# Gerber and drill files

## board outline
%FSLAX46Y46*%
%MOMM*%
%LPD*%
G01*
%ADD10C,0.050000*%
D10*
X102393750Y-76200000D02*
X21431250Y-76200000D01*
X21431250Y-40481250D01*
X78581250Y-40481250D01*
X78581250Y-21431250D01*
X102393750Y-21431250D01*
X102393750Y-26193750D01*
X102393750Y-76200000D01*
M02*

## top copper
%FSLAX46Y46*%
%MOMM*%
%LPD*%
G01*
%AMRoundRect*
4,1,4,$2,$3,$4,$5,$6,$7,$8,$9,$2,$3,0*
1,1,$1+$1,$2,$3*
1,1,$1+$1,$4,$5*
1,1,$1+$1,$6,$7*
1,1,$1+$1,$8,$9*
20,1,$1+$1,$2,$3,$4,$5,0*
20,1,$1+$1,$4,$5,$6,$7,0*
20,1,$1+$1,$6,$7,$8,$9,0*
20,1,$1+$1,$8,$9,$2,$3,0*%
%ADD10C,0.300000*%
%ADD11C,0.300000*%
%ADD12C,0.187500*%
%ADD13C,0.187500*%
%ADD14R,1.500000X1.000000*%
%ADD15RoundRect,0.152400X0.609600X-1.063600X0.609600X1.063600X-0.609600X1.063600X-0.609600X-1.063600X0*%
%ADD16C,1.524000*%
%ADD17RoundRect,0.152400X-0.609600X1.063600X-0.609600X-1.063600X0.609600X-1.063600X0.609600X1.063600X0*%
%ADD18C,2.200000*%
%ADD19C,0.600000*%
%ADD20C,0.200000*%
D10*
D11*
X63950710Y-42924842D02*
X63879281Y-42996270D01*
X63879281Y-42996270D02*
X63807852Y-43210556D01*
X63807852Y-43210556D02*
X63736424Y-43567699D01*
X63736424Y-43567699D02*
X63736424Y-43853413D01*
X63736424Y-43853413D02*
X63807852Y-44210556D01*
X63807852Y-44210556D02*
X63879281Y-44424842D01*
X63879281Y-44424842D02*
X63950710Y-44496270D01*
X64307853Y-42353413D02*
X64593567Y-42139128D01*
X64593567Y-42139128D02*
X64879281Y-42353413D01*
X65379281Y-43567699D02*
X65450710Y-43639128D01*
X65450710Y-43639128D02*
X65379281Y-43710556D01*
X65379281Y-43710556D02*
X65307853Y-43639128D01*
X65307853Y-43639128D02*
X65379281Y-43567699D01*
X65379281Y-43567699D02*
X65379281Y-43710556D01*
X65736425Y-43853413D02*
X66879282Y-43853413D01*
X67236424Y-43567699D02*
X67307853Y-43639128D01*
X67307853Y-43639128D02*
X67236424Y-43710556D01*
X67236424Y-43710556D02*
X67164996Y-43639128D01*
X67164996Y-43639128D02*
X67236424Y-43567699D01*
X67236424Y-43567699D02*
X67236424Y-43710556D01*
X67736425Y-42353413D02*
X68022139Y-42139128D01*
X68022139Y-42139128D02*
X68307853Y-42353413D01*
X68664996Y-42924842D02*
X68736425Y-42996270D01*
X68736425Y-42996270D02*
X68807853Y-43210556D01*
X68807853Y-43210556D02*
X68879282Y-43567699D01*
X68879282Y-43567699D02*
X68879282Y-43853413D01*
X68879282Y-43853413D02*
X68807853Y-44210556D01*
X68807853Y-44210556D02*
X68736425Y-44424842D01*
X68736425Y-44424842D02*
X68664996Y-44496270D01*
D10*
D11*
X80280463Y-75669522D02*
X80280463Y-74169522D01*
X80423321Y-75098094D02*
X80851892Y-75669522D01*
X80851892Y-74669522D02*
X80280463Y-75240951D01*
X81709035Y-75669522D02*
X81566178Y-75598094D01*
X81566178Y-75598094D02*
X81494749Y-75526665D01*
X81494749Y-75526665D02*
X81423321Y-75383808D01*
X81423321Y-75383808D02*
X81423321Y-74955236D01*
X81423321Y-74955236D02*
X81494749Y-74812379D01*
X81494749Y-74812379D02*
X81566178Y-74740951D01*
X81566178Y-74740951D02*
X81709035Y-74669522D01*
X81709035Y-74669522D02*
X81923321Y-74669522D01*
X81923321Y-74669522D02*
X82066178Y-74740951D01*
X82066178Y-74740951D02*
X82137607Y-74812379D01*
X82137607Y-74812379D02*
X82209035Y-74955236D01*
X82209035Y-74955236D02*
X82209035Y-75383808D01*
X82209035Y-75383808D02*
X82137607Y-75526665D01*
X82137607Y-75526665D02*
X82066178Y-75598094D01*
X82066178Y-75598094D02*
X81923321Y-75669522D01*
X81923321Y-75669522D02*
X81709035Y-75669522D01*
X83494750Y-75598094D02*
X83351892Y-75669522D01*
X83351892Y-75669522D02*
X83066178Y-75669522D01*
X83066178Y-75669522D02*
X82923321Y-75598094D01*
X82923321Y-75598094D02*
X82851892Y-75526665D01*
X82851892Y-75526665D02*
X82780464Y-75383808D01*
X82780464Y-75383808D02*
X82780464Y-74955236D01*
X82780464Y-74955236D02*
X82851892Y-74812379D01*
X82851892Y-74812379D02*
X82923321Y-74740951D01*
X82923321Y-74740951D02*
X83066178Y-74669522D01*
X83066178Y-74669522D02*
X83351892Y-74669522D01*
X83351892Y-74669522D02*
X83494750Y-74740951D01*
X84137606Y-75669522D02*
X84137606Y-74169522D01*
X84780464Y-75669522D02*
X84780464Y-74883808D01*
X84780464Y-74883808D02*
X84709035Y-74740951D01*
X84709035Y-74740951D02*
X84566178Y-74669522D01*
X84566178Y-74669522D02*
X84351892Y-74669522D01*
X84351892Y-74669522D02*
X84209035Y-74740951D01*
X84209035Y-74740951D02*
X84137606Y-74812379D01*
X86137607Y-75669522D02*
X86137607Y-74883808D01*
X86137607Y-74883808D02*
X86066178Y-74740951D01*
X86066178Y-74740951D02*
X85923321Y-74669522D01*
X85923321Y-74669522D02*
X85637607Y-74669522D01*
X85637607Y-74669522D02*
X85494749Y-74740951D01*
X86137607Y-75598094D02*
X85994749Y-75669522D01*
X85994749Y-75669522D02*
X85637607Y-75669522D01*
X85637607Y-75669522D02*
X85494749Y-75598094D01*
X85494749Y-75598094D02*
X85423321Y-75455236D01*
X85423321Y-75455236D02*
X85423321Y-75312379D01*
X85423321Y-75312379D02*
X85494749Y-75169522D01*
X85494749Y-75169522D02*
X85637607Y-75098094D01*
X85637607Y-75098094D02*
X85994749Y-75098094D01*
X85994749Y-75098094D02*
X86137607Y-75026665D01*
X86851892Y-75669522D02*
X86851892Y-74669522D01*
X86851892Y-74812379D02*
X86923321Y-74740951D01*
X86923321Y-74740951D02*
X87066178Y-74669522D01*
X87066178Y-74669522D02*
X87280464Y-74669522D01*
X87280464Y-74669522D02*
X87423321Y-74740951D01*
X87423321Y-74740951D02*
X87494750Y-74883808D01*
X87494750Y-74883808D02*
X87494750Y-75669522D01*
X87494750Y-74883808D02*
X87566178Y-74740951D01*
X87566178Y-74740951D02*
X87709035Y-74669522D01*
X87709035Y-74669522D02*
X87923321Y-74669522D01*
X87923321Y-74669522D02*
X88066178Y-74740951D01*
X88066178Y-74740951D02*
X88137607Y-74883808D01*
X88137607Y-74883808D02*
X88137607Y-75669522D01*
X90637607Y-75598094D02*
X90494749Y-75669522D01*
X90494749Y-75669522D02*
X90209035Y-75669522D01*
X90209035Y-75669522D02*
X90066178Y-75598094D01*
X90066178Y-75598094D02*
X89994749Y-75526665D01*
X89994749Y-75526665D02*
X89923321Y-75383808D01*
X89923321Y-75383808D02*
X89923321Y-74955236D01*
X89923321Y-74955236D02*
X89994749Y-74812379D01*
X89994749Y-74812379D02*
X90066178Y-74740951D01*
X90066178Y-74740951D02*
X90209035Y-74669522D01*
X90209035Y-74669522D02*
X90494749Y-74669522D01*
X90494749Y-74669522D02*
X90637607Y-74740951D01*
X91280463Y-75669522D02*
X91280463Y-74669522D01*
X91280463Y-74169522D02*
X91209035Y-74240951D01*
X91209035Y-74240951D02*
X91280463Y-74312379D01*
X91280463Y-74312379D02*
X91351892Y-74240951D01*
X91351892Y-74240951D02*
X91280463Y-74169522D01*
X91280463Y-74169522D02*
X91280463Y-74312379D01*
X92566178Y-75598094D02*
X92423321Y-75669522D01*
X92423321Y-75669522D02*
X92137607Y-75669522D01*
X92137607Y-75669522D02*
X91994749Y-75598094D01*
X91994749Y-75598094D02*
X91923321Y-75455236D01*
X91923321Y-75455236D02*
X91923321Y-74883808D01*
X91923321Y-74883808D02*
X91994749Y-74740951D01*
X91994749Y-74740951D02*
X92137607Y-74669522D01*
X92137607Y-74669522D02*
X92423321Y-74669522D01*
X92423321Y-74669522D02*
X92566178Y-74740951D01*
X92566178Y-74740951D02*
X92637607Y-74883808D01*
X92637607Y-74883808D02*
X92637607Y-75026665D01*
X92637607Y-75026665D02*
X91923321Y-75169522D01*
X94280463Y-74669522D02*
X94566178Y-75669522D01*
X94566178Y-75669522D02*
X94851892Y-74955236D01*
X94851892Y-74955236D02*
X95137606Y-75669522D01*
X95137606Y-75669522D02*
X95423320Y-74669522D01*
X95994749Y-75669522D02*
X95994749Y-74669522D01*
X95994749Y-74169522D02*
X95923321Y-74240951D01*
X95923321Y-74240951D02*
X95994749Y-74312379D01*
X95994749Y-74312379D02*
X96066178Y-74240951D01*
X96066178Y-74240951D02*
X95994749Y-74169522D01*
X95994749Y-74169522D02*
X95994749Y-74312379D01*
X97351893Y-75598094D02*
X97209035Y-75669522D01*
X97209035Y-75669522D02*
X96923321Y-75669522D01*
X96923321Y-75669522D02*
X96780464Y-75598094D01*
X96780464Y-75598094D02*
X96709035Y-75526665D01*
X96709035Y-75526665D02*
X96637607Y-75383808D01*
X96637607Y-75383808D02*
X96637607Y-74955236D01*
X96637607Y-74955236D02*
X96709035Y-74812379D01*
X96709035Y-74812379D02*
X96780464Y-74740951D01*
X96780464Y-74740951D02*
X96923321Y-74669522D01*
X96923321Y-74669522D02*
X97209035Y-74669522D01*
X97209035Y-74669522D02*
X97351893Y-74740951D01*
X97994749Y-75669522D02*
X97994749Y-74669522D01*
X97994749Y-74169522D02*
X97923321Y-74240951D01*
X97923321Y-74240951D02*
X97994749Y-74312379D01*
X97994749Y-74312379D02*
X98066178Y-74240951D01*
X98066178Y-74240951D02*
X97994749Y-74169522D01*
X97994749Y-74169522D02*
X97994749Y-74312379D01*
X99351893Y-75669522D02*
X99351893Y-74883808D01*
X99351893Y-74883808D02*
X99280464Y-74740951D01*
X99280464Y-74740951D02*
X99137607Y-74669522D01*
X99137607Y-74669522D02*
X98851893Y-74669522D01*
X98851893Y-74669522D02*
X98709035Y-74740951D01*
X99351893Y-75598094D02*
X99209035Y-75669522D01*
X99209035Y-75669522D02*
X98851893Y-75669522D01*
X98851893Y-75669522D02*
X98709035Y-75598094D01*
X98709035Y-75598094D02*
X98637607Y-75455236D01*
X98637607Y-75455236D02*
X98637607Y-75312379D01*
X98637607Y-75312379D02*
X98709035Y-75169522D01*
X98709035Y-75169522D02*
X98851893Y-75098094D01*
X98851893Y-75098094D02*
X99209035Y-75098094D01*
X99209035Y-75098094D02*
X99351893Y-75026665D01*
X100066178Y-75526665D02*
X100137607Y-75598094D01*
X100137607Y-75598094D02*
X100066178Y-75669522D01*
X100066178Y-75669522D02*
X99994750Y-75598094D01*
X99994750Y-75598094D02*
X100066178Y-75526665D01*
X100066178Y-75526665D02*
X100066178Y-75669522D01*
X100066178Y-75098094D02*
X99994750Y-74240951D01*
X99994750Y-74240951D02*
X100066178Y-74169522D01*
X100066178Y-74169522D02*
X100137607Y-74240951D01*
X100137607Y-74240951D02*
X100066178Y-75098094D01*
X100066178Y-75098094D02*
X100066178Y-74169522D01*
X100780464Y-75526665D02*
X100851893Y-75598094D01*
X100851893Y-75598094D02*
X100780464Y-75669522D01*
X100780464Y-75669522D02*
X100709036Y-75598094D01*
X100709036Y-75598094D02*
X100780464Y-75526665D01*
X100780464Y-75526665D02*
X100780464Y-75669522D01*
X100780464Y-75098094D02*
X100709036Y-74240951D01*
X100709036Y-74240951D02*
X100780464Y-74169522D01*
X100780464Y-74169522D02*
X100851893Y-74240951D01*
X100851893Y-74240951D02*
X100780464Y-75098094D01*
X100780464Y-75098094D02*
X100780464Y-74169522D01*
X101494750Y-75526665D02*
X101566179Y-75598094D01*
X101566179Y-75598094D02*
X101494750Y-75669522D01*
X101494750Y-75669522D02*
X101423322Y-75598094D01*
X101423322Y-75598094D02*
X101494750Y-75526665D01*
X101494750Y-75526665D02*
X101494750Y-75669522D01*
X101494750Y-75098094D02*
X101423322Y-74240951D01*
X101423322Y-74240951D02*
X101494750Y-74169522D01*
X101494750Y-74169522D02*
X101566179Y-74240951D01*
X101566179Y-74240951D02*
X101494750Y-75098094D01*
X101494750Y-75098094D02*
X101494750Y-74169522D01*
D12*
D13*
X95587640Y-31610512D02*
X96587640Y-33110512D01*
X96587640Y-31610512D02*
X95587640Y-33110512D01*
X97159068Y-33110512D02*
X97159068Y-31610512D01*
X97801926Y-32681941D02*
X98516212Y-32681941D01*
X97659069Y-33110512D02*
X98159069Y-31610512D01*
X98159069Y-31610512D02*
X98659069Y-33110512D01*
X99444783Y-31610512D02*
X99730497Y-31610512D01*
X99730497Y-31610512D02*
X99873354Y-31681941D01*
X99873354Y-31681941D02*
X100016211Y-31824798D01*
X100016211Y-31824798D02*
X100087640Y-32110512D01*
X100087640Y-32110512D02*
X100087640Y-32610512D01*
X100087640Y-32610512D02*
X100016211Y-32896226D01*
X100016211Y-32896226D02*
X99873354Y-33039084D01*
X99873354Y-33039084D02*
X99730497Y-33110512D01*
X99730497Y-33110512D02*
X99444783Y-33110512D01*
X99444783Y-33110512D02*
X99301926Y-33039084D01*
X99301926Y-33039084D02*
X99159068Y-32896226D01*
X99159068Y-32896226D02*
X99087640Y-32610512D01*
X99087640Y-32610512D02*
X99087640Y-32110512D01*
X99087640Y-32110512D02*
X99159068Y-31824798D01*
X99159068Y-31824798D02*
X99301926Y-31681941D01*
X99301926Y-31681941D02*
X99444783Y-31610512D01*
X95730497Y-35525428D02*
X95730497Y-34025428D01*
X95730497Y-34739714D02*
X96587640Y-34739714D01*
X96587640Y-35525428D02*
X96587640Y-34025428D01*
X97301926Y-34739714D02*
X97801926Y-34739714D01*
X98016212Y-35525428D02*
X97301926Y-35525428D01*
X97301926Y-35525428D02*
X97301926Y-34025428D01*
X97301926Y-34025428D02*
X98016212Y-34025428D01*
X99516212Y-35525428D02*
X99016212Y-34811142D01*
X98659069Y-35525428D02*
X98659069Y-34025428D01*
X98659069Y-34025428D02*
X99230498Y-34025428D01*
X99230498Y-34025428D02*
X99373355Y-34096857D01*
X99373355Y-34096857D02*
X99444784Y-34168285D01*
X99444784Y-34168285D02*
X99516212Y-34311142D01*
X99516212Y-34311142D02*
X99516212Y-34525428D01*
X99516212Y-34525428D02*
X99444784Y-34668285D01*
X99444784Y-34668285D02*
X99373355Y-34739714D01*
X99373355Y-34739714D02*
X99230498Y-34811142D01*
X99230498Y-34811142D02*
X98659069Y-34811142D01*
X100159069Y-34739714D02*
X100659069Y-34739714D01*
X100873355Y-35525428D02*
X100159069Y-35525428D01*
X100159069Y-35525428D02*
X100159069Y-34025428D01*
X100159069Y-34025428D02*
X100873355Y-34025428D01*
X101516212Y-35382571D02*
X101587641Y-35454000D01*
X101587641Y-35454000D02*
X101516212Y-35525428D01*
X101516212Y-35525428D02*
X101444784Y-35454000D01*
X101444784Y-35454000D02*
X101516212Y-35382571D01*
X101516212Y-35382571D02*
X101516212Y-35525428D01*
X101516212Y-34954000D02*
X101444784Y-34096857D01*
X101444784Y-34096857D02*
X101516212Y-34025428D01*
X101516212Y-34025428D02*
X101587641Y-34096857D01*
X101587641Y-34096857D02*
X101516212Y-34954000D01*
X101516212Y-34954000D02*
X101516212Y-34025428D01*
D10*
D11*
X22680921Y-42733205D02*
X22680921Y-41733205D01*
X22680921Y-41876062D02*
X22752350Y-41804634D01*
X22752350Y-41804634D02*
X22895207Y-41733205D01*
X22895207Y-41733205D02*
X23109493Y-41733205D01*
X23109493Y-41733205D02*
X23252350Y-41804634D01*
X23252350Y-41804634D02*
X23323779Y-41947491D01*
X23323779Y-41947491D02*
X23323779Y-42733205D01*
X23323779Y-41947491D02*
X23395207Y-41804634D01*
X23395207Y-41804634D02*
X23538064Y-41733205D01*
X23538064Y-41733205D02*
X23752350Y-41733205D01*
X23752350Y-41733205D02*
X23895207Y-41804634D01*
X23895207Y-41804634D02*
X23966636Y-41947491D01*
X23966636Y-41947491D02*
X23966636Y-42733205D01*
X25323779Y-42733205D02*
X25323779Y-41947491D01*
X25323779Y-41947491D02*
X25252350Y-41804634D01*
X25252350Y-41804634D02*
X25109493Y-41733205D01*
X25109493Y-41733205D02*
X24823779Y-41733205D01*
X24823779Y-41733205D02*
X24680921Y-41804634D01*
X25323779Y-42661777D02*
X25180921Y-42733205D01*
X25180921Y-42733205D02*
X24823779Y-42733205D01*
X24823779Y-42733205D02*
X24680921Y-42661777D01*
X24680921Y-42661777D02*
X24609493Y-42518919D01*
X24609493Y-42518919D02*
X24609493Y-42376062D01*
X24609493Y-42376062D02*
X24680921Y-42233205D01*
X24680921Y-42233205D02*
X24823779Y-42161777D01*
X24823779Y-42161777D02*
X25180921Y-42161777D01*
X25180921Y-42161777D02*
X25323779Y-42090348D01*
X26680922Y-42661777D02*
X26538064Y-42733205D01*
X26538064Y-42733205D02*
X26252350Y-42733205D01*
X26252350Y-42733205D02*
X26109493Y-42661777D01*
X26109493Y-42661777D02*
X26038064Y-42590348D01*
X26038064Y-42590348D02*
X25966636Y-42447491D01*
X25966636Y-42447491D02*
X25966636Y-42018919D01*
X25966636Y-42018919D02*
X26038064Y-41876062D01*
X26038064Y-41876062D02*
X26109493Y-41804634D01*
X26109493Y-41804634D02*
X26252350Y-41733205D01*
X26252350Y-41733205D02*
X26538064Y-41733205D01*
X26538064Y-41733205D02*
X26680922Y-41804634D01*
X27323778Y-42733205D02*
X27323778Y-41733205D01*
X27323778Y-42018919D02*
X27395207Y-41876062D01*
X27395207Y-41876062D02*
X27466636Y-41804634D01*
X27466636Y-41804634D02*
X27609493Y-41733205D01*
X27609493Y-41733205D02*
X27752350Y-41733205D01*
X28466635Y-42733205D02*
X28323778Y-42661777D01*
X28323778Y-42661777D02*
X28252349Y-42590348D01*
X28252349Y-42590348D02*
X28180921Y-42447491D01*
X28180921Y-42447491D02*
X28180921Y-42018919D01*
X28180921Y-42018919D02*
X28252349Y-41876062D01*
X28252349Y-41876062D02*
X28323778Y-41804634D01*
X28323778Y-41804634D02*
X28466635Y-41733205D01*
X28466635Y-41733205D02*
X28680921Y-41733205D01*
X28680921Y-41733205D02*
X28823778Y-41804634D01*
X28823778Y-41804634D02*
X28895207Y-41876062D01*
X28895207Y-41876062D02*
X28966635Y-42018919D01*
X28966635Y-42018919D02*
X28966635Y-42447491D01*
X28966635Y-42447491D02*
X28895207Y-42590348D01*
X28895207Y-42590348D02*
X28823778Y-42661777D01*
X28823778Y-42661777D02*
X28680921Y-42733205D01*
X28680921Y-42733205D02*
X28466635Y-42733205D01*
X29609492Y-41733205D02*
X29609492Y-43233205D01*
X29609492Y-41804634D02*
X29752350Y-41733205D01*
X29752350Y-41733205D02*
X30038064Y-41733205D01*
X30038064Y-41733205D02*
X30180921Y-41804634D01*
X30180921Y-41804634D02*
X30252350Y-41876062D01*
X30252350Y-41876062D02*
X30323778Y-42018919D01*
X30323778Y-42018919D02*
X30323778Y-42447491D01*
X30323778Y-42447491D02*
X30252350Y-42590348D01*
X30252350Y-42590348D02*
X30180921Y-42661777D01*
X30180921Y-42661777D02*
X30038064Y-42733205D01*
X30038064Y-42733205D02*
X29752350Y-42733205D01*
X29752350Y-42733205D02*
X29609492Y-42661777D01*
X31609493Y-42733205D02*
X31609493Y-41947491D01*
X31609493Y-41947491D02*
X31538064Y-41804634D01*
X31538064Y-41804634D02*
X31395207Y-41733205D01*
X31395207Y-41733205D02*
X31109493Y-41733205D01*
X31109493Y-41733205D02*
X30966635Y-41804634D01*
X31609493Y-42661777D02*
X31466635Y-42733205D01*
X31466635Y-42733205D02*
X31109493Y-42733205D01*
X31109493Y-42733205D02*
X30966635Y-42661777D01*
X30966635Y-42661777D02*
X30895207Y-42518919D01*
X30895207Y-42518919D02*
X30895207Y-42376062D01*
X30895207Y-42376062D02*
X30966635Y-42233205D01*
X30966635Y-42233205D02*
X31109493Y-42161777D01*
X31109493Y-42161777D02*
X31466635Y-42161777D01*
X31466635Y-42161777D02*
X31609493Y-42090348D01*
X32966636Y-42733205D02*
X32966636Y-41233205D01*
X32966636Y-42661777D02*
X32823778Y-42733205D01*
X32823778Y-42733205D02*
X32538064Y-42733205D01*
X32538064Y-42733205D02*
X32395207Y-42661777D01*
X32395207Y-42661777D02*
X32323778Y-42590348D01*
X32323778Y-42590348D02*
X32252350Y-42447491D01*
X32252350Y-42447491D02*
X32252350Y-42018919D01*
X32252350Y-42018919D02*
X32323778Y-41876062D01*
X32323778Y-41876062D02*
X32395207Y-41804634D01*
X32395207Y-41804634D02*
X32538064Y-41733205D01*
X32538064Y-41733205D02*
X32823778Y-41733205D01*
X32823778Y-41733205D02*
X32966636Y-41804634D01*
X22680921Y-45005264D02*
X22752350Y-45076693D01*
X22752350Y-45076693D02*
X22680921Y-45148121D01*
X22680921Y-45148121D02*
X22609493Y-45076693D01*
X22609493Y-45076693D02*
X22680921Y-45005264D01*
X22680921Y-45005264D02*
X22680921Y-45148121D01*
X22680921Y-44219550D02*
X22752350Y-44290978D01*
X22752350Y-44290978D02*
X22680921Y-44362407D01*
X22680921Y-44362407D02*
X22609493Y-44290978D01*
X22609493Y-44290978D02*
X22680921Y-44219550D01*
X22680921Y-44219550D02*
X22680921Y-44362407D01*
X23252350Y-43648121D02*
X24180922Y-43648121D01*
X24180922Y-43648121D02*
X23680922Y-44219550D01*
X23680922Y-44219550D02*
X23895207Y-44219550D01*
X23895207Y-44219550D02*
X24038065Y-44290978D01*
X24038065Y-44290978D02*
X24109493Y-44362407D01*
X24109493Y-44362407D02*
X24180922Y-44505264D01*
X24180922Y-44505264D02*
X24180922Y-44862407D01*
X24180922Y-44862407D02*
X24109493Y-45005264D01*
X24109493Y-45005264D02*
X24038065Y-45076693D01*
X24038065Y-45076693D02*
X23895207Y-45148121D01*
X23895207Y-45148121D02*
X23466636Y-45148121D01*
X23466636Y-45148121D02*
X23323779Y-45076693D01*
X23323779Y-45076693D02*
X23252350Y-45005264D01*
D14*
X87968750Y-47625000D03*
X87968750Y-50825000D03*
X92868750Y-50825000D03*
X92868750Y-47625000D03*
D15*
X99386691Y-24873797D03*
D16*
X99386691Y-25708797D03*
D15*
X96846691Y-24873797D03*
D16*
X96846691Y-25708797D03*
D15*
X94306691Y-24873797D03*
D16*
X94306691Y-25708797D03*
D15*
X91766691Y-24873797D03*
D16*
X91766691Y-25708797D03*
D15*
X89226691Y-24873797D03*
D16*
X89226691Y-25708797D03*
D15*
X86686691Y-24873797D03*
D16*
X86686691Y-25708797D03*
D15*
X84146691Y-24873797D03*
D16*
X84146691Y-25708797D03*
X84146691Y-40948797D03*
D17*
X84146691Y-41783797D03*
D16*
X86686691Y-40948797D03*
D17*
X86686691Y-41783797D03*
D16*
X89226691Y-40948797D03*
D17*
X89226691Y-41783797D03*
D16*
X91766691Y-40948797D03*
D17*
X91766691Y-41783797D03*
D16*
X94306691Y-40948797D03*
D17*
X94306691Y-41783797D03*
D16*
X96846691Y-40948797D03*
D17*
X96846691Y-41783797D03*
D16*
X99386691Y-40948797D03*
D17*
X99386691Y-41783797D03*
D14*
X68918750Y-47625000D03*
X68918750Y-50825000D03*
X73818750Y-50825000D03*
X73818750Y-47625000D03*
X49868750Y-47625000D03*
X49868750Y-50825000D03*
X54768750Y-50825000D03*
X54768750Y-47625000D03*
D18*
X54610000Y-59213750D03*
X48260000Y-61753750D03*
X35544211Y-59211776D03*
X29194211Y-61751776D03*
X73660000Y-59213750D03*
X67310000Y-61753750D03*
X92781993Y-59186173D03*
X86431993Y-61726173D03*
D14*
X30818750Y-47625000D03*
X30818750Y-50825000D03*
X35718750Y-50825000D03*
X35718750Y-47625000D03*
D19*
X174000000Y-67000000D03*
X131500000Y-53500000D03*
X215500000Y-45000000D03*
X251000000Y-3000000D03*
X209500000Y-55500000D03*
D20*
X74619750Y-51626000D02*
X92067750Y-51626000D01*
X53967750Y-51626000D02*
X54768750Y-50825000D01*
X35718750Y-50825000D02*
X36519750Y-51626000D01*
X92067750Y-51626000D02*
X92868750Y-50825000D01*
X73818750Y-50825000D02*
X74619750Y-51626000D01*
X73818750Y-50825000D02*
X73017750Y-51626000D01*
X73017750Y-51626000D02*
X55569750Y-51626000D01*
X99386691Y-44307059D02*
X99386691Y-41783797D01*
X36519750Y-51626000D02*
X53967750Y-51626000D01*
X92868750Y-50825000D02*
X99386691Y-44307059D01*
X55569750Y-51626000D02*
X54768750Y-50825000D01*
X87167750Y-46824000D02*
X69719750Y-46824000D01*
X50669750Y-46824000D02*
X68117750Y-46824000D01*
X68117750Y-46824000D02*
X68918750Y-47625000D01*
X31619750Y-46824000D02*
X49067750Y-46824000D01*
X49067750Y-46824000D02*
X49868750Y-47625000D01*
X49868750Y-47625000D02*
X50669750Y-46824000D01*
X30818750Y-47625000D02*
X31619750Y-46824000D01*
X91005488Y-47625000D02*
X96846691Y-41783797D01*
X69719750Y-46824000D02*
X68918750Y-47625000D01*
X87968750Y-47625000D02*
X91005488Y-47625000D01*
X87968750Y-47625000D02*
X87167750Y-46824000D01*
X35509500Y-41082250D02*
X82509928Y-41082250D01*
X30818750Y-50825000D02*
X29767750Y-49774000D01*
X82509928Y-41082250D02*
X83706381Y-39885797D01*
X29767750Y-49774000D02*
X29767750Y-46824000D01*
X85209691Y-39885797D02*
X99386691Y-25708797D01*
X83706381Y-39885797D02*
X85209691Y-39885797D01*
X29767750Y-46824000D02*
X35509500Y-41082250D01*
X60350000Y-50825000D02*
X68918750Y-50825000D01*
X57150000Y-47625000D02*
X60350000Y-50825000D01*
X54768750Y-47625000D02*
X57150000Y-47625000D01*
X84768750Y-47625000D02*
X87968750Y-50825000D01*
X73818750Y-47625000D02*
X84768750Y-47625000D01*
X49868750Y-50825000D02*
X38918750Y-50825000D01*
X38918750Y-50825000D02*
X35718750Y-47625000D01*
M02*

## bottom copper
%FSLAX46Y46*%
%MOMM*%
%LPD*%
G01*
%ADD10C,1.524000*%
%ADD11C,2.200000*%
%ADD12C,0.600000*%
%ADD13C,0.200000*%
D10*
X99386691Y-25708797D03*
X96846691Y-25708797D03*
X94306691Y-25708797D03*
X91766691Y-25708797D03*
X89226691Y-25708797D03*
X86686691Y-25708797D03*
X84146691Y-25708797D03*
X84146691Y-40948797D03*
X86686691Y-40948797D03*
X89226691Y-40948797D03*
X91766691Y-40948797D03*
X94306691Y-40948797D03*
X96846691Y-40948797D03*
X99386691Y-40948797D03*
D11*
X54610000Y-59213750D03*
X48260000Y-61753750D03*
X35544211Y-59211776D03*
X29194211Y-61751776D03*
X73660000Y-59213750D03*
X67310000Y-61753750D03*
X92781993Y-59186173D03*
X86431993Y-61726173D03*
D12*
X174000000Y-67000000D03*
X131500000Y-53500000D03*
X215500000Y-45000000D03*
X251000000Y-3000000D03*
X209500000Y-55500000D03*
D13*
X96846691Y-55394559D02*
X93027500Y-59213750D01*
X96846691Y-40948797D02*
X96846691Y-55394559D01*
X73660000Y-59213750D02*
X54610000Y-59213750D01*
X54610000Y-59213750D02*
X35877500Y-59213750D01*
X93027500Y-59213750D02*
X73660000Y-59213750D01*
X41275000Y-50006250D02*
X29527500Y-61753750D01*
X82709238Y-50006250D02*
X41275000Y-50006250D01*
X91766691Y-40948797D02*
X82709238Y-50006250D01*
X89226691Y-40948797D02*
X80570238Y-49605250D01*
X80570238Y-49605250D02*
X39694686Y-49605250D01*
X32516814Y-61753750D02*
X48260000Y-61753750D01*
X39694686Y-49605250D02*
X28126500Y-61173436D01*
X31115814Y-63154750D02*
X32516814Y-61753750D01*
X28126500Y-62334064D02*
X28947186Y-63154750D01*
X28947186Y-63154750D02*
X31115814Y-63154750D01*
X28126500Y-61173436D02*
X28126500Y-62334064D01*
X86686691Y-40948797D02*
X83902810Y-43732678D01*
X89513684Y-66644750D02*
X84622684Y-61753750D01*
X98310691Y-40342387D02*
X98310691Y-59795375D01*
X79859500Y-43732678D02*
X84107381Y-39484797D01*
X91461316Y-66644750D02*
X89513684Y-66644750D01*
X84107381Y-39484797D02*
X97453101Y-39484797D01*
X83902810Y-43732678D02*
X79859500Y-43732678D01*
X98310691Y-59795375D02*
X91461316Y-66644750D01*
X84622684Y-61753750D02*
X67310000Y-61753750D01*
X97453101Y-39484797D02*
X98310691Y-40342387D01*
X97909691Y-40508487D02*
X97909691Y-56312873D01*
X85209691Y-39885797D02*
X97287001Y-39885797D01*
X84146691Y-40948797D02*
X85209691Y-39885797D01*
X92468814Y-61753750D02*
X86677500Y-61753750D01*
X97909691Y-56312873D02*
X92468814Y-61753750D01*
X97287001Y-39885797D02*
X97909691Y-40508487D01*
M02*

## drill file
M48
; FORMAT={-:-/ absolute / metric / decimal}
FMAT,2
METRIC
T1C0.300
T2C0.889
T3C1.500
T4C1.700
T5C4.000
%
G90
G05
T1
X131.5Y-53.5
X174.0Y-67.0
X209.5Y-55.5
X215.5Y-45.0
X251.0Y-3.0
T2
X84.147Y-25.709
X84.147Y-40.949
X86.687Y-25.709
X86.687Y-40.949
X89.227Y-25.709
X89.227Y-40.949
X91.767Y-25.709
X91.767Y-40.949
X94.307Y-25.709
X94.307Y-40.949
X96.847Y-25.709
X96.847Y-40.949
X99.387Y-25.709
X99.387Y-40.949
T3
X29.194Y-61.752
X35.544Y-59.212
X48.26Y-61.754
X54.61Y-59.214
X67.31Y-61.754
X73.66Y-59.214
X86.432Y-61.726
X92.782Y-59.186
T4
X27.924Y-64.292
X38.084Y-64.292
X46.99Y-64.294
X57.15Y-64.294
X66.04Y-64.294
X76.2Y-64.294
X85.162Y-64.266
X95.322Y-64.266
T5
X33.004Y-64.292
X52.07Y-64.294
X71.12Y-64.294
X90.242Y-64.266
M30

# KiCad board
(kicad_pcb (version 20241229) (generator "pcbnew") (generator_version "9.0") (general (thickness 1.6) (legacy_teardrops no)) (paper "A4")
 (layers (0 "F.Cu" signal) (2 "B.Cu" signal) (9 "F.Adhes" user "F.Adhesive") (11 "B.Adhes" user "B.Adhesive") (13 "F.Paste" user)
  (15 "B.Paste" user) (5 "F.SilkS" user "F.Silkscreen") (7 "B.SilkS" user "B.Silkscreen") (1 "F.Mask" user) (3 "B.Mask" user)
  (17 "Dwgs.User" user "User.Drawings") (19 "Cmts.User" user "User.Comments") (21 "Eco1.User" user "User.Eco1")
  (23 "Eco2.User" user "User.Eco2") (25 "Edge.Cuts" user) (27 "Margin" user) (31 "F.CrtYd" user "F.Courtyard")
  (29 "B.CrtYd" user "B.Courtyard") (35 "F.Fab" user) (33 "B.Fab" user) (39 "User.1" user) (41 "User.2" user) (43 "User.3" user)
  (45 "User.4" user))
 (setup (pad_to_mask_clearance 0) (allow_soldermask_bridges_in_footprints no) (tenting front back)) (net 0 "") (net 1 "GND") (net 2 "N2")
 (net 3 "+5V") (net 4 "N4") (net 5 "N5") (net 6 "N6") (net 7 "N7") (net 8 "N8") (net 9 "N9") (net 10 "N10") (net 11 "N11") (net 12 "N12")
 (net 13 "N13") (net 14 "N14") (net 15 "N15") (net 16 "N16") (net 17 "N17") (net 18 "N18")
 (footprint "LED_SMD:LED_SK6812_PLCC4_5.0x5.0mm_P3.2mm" (layer "F.Cu") (at 90.41875 49.225)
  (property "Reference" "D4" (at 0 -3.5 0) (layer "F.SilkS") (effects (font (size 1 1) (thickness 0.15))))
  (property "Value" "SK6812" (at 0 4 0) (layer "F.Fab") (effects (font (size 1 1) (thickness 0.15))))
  (pad "1" smd rect (at -2.45 -1.6 180) (size 1.5 1) (layers "F.Cu" "F.Mask" "F.Paste") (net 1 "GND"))
  (pad "2" smd rect (at -2.45 1.6 180) (size 1.5 1) (layers "F.Cu" "F.Mask" "F.Paste") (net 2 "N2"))
  (pad "3" smd rect (at 2.45 1.6 180) (size 1.5 1) (layers "F.Cu" "F.Mask" "F.Paste") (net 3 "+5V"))
  (pad "4" smd rect (at 2.45 -1.6 180) (size 1.5 1) (layers "F.Cu" "F.Mask" "F.Paste") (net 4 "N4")))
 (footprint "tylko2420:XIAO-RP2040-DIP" (layer "F.Cu") (at 91.766691 33.328797 -90)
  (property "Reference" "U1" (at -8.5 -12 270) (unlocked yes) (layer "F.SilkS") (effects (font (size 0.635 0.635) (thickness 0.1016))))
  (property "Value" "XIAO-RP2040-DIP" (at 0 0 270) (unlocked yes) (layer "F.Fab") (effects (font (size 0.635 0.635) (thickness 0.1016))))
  (pad "1" smd roundrect (at -8.455 -7.62 90) (size 2.432 1.524) (layers "F.Cu" "F.Mask") (roundrect_rratio 0.1) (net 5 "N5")
   (thermal_bridge_angle 45))
  (pad "1" thru_hole circle (at -7.62 -7.62 90) (size 1.524 1.524) (drill 0.889) (layers "*.Cu" "*.Mask") (remove_unused_layers no)
   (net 5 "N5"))
  (pad "2" smd roundrect (at -8.455 -5.08 90) (size 2.432 1.524) (layers "F.Cu" "F.Mask") (roundrect_rratio 0.1) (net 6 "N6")
   (thermal_bridge_angle 45))
  (pad "2" thru_hole circle (at -7.62 -5.08 90) (size 1.524 1.524) (drill 0.889) (layers "*.Cu" "*.Mask") (remove_unused_layers no)
   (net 6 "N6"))
  (pad "3" smd roundrect (at -8.455 -2.54 90) (size 2.432 1.524) (layers "F.Cu" "F.Mask") (roundrect_rratio 0.1) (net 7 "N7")
   (thermal_bridge_angle 45))
  (pad "3" thru_hole circle (at -7.62 -2.54 90) (size 1.524 1.524) (drill 0.889) (layers "*.Cu" "*.Mask") (remove_unused_layers no)
   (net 7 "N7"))
  (pad "4" smd roundrect (at -8.455 0 90) (size 2.432 1.524) (layers "F.Cu" "F.Mask") (roundrect_rratio 0.1) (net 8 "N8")
   (thermal_bridge_angle 45))
  (pad "4" thru_hole circle (at -7.62 0 90) (size 1.524 1.524) (drill 0.889) (layers "*.Cu" "*.Mask") (remove_unused_layers no) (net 8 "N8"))
  (pad "5" smd roundrect (at -8.455 2.54 90) (size 2.432 1.524) (layers "F.Cu" "F.Mask") (roundrect_rratio 0.1) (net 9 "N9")
   (thermal_bridge_angle 45))
  (pad "5" thru_hole circle (at -7.62 2.54 90) (size 1.524 1.524) (drill 0.889) (layers "*.Cu" "*.Mask") (remove_unused_layers no)
   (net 9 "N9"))
  (pad "6" smd roundrect (at -8.455 5.08 90) (size 2.432 1.524) (layers "F.Cu" "F.Mask") (roundrect_rratio 0.1) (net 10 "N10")
   (thermal_bridge_angle 45))
  (pad "6" thru_hole circle (at -7.62 5.08 90) (size 1.524 1.524) (drill 0.889) (layers "*.Cu" "*.Mask") (remove_unused_layers no)
   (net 10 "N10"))
  (pad "7" smd roundrect (at -8.455 7.62 90) (size 2.432 1.524) (layers "F.Cu" "F.Mask") (roundrect_rratio 0.1) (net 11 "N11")
   (thermal_bridge_angle 45))
  (pad "7" thru_hole circle (at -7.62 7.62 90) (size 1.524 1.524) (drill 0.889) (layers "*.Cu" "*.Mask") (remove_unused_layers no)
   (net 11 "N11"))
  (pad "8" thru_hole circle (at 7.62 7.62 270) (size 1.524 1.524) (drill 0.889) (layers "*.Cu" "*.Mask") (remove_unused_layers no)
   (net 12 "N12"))
  (pad "8" smd roundrect (at 8.455 7.62 270) (size 2.432 1.524) (layers "F.Cu" "F.Mask") (roundrect_rratio 0.1) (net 12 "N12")
   (thermal_bridge_angle 45))
  (pad "9" thru_hole circle (at 7.62 5.08 270) (size 1.524 1.524) (drill 0.889) (layers "*.Cu" "*.Mask") (remove_unused_layers no)
   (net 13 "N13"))
  (pad "9" smd roundrect (at 8.455 5.08 270) (size 2.432 1.524) (layers "F.Cu" "F.Mask") (roundrect_rratio 0.1) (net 13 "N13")
   (thermal_bridge_angle 45))
  (pad "10" thru_hole circle (at 7.62 2.54 270) (size 1.524 1.524) (drill 0.889) (layers "*.Cu" "*.Mask") (remove_unused_layers no)
   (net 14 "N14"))
  (pad "10" smd roundrect (at 8.455 2.54 270) (size 2.432 1.524) (layers "F.Cu" "F.Mask") (roundrect_rratio 0.1) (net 14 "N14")
   (thermal_bridge_angle 45))
  (pad "11" thru_hole circle (at 7.62 0 270) (size 1.524 1.524) (drill 0.889) (layers "*.Cu" "*.Mask") (remove_unused_layers no)
   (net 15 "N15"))
  (pad "11" smd roundrect (at 8.455 0 270) (size 2.432 1.524) (layers "F.Cu" "F.Mask") (roundrect_rratio 0.1) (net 15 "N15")
   (thermal_bridge_angle 45))
  (pad "12" thru_hole circle (at 7.62 -2.54 270) (size 1.524 1.524) (drill 0.889) (layers "*.Cu" "*.Mask") (remove_unused_layers no)
   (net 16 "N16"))
  (pad "12" smd roundrect (at 8.455 -2.54 270) (size 2.432 1.524) (layers "F.Cu" "F.Mask") (roundrect_rratio 0.1) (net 16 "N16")
   (thermal_bridge_angle 45))
  (pad "13" thru_hole circle (at 7.62 -5.08 270) (size 1.524 1.524) (drill 0.889) (layers "*.Cu" "*.Mask") (remove_unused_layers no)
   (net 1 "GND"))
  (pad "13" smd roundrect (at 8.455 -5.08 270) (size 2.432 1.524) (layers "F.Cu" "F.Mask") (roundrect_rratio 0.1) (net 1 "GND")
   (thermal_bridge_angle 45))
  (pad "14" thru_hole circle (at 7.62 -7.62 270) (size 1.524 1.524) (drill 0.889) (layers "*.Cu" "*.Mask") (remove_unused_layers no)
   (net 3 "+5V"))
  (pad "14" smd roundrect (at 8.455 -7.62 270) (size 2.432 1.524) (layers "F.Cu" "F.Mask") (roundrect_rratio 0.1) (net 3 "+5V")
   (thermal_bridge_angle 45)))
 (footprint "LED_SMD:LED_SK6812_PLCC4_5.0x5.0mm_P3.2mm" (layer "F.Cu") (at 71.36875 49.225)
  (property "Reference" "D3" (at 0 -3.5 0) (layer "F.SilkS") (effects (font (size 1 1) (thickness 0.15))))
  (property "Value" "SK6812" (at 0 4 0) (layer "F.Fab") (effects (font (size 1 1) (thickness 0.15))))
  (pad "1" smd rect (at -2.45 -1.6 180) (size 1.5 1) (layers "F.Cu" "F.Mask" "F.Paste") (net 1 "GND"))
  (pad "2" smd rect (at -2.45 1.6 180) (size 1.5 1) (layers "F.Cu" "F.Mask" "F.Paste") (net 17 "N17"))
  (pad "3" smd rect (at 2.45 1.6 180) (size 1.5 1) (layers "F.Cu" "F.Mask" "F.Paste") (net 3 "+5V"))
  (pad "4" smd rect (at 2.45 -1.6 180) (size 1.5 1) (layers "F.Cu" "F.Mask" "F.Paste") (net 2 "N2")))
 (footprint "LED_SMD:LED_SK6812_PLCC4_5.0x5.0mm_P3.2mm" (layer "F.Cu") (at 52.31875 49.225)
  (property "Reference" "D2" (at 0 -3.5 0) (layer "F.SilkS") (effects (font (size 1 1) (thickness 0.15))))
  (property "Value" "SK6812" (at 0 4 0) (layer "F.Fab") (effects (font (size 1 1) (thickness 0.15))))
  (pad "1" smd rect (at -2.45 -1.6 180) (size 1.5 1) (layers "F.Cu" "F.Mask" "F.Paste") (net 1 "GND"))
  (pad "2" smd rect (at -2.45 1.6 180) (size 1.5 1) (layers "F.Cu" "F.Mask" "F.Paste") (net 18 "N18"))
  (pad "3" smd rect (at 2.45 1.6 180) (size 1.5 1) (layers "F.Cu" "F.Mask" "F.Paste") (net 3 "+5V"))
  (pad "4" smd rect (at 2.45 -1.6 180) (size 1.5 1) (layers "F.Cu" "F.Mask" "F.Paste") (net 17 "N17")))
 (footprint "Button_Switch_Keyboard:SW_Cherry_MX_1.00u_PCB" (layer "F.Cu") (at 54.61 59.21375)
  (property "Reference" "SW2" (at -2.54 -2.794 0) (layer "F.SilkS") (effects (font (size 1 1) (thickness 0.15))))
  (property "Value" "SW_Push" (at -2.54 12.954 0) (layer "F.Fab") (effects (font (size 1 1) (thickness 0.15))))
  (pad "" np_thru_hole circle (at -7.62 5.08) (size 1.7 1.7) (drill 1.7) (layers "*.Cu" "*.Mask"))
  (pad "" np_thru_hole circle (at -2.54 5.08) (size 4 4) (drill 4) (layers "*.Cu" "*.Mask"))
  (pad "" np_thru_hole circle (at 2.54 5.08) (size 1.7 1.7) (drill 1.7) (layers "*.Cu" "*.Mask"))
  (pad "1" thru_hole circle (at 0 0) (size 2.2 2.2) (drill 1.5) (layers "*.Cu" "*.Mask") (remove_unused_layers no) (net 1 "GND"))
  (pad "2" thru_hole circle (at -6.35 2.54) (size 2.2 2.2) (drill 1.5) (layers "*.Cu" "*.Mask") (remove_unused_layers no) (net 14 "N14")))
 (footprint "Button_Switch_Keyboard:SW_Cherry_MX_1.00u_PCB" (layer "F.Cu") (at 35.544211 59.211776)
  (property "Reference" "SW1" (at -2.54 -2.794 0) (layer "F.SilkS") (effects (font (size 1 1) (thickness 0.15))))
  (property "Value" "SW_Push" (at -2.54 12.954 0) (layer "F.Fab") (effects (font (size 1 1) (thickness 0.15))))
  (pad "" np_thru_hole circle (at -7.62 5.08) (size 1.7 1.7) (drill 1.7) (layers "*.Cu" "*.Mask"))
  (pad "" np_thru_hole circle (at -2.54 5.08) (size 4 4) (drill 4) (layers "*.Cu" "*.Mask"))
  (pad "" np_thru_hole circle (at 2.54 5.08) (size 1.7 1.7) (drill 1.7) (layers "*.Cu" "*.Mask"))
  (pad "1" thru_hole circle (at 0 0) (size 2.2 2.2) (drill 1.5) (layers "*.Cu" "*.Mask") (remove_unused_layers no) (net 1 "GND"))
  (pad "2" thru_hole circle (at -6.35 2.54) (size 2.2 2.2) (drill 1.5) (layers "*.Cu" "*.Mask") (remove_unused_layers no) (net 15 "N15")))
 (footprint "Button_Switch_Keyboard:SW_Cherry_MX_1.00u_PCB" (layer "F.Cu") (at 73.66 59.21375)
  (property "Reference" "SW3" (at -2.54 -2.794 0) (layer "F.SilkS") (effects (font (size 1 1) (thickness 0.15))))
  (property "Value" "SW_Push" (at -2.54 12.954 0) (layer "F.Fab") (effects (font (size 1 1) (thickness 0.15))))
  (pad "" np_thru_hole circle (at -7.62 5.08) (size 1.7 1.7) (drill 1.7) (layers "*.Cu" "*.Mask"))
  (pad "" np_thru_hole circle (at -2.54 5.08) (size 4 4) (drill 4) (layers "*.Cu" "*.Mask"))
  (pad "" np_thru_hole circle (at 2.54 5.08) (size 1.7 1.7) (drill 1.7) (layers "*.Cu" "*.Mask"))
  (pad "1" thru_hole circle (at 0 0) (size 2.2 2.2) (drill 1.5) (layers "*.Cu" "*.Mask") (remove_unused_layers no) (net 1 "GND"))
  (pad "2" thru_hole circle (at -6.35 2.54) (size 2.2 2.2) (drill 1.5) (layers "*.Cu" "*.Mask") (remove_unused_layers no) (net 13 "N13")))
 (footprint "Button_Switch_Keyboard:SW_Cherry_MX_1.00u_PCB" (layer "F.Cu") (at 92.781993 59.186173)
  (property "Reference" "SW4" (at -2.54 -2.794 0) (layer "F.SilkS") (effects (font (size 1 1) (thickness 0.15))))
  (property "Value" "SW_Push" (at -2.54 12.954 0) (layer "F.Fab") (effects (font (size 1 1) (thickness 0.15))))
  (pad "" np_thru_hole circle (at -7.62 5.08) (size 1.7 1.7) (drill 1.7) (layers "*.Cu" "*.Mask"))
  (pad "" np_thru_hole circle (at -2.54 5.08) (size 4 4) (drill 4) (layers "*.Cu" "*.Mask"))
  (pad "" np_thru_hole circle (at 2.54 5.08) (size 1.7 1.7) (drill 1.7) (layers "*.Cu" "*.Mask"))
  (pad "1" thru_hole circle (at 0 0) (size 2.2 2.2) (drill 1.5) (layers "*.Cu" "*.Mask") (remove_unused_layers no) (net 1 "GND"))
  (pad "2" thru_hole circle (at -6.35 2.54) (size 2.2 2.2) (drill 1.5) (layers "*.Cu" "*.Mask") (remove_unused_layers no) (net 12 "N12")))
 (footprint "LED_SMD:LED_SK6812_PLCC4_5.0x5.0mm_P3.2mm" (layer "F.Cu") (at 33.26875 49.225)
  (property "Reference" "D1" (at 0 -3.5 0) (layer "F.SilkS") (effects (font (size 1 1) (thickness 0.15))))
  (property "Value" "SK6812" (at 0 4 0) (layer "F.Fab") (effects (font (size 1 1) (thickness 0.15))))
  (pad "1" smd rect (at -2.45 -1.6 180) (size 1.5 1) (layers "F.Cu" "F.Mask" "F.Paste") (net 1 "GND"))
  (pad "2" smd rect (at -2.45 1.6 180) (size 1.5 1) (layers "F.Cu" "F.Mask" "F.Paste") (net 5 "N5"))
  (pad "3" smd rect (at 2.45 1.6 180) (size 1.5 1) (layers "F.Cu" "F.Mask" "F.Paste") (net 3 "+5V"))
  (pad "4" smd rect (at 2.45 -1.6 180) (size 1.5 1) (layers "F.Cu" "F.Mask" "F.Paste") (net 18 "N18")))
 (gr_poly
  (pts (xy 102.39375 76.2) (xy 21.43125 76.2) (xy 21.43125 40.48125) (xy 78.58125 40.48125) (xy 78.58125 21.43125) (xy 102.39375 21.43125)
   (xy 102.39375 26.19375))
  (stroke (width 0.05) (type solid)) (fill no) (layer "Edge.Cuts"))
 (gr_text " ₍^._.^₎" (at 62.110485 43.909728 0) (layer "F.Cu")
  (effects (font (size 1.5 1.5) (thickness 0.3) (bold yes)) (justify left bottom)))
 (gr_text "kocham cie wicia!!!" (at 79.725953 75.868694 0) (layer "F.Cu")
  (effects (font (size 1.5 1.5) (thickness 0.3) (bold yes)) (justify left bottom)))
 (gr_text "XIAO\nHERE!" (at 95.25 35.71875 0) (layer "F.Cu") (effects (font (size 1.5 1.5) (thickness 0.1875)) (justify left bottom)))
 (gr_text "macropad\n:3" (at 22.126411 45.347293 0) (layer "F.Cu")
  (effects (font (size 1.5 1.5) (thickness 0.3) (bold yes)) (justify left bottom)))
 (via (at 174 67) (size 0.6) (drill 0.3) (layers "F.Cu" "B.Cu") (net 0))
 (via (at 131.5 53.5) (size 0.6) (drill 0.3) (layers "F.Cu" "B.Cu") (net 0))
 (via (at 215.5 45) (size 0.6) (drill 0.3) (layers "F.Cu" "B.Cu") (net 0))
 (via (at 251 3) (size 0.6) (drill 0.3) (layers "F.Cu" "B.Cu") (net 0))
 (via (at 209.5 55.5) (size 0.6) (drill 0.3) (layers "F.Cu" "B.Cu") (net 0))
 (segment (start 74.61975 51.626) (end 92.06775 51.626) (width 0.2) (layer "F.Cu") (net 3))
 (segment (start 53.96775 51.626) (end 54.76875 50.825) (width 0.2) (layer "F.Cu") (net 3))
 (segment (start 35.71875 50.825) (end 36.51975 51.626) (width 0.2) (layer "F.Cu") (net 3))
 (segment (start 92.06775 51.626) (end 92.86875 50.825) (width 0.2) (layer "F.Cu") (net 3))
 (segment (start 73.81875 50.825) (end 74.61975 51.626) (width 0.2) (layer "F.Cu") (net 3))
 (segment (start 73.81875 50.825) (end 73.01775 51.626) (width 0.2) (layer "F.Cu") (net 3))
 (segment (start 73.01775 51.626) (end 55.56975 51.626) (width 0.2) (layer "F.Cu") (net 3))
 (segment (start 99.386691 44.307059) (end 99.386691 41.783797) (width 0.2) (layer "F.Cu") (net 3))
 (segment (start 36.51975 51.626) (end 53.96775 51.626) (width 0.2) (layer "F.Cu") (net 3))
 (segment (start 92.86875 50.825) (end 99.386691 44.307059) (width 0.2) (layer "F.Cu") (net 3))
 (segment (start 55.56975 51.626) (end 54.76875 50.825) (width 0.2) (layer "F.Cu") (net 3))
 (segment (start 87.16775 46.824) (end 69.71975 46.824) (width 0.2) (layer "F.Cu") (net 1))
 (segment (start 50.66975 46.824) (end 68.11775 46.824) (width 0.2) (layer "F.Cu") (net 1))
 (segment (start 68.11775 46.824) (end 68.91875 47.625) (width 0.2) (layer "F.Cu") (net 1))
 (segment (start 31.61975 46.824) (end 49.06775 46.824) (width 0.2) (layer "F.Cu") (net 1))
 (segment (start 49.06775 46.824) (end 49.86875 47.625) (width 0.2) (layer "F.Cu") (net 1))
 (segment (start 49.86875 47.625) (end 50.66975 46.824) (width 0.2) (layer "F.Cu") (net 1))
 (segment (start 30.81875 47.625) (end 31.61975 46.824) (width 0.2) (layer "F.Cu") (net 1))
 (segment (start 91.005488 47.625) (end 96.846691 41.783797) (width 0.2) (layer "F.Cu") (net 1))
 (segment (start 69.71975 46.824) (end 68.91875 47.625) (width 0.2) (layer "F.Cu") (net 1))
 (segment (start 87.96875 47.625) (end 91.005488 47.625) (width 0.2) (layer "F.Cu") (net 1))
 (segment (start 87.96875 47.625) (end 87.16775 46.824) (width 0.2) (layer "F.Cu") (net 1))
 (segment (start 96.846691 55.394559) (end 93.0275 59.21375) (width 0.2) (layer "B.Cu") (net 1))
 (segment (start 96.846691 40.948797) (end 96.846691 55.394559) (width 0.2) (layer "B.Cu") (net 1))
 (segment (start 73.66 59.21375) (end 54.61 59.21375) (width 0.2) (layer "B.Cu") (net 1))
 (segment (start 54.61 59.21375) (end 35.8775 59.21375) (width 0.2) (layer "B.Cu") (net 1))
 (segment (start 93.0275 59.21375) (end 73.66 59.21375) (width 0.2) (layer "B.Cu") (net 1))
 (segment (start 35.5095 41.08225) (end 82.509928 41.08225) (width 0.2) (layer "F.Cu") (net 5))
 (segment (start 30.81875 50.825) (end 29.76775 49.774) (width 0.2) (layer "F.Cu") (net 5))
 (segment (start 82.509928 41.08225) (end 83.706381 39.885797) (width 0.2) (layer "F.Cu") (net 5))
 (segment (start 29.76775 49.774) (end 29.76775 46.824) (width 0.2) (layer "F.Cu") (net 5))
 (segment (start 85.209691 39.885797) (end 99.386691 25.708797) (width 0.2) (layer "F.Cu") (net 5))
 (segment (start 83.706381 39.885797) (end 85.209691 39.885797) (width 0.2) (layer "F.Cu") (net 5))
 (segment (start 29.76775 46.824) (end 35.5095 41.08225) (width 0.2) (layer "F.Cu") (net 5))
 (segment (start 60.35 50.825) (end 68.91875 50.825) (width 0.2) (layer "F.Cu") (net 17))
 (segment (start 57.15 47.625) (end 60.35 50.825) (width 0.2) (layer "F.Cu") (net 17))
 (segment (start 54.76875 47.625) (end 57.15 47.625) (width 0.2) (layer "F.Cu") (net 17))
 (segment (start 84.76875 47.625) (end 87.96875 50.825) (width 0.2) (layer "F.Cu") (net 2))
 (segment (start 73.81875 47.625) (end 84.76875 47.625) (width 0.2) (layer "F.Cu") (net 2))
 (segment (start 41.275 50.00625) (end 29.5275 61.75375) (width 0.2) (layer "B.Cu") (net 15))
 (segment (start 82.709238 50.00625) (end 41.275 50.00625) (width 0.2) (layer "B.Cu") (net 15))
 (segment (start 91.766691 40.948797) (end 82.709238 50.00625) (width 0.2) (layer "B.Cu") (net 15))
 (segment (start 89.226691 40.948797) (end 80.570238 49.60525) (width 0.2) (layer "B.Cu") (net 14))
 (segment (start 80.570238 49.60525) (end 39.694686 49.60525) (width 0.2) (layer "B.Cu") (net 14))
 (segment (start 32.516814 61.75375) (end 48.26 61.75375) (width 0.2) (layer "B.Cu") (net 14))
 (segment (start 39.694686 49.60525) (end 28.1265 61.173436) (width 0.2) (layer "B.Cu") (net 14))
 (segment (start 31.115814 63.15475) (end 32.516814 61.75375) (width 0.2) (layer "B.Cu") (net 14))
 (segment (start 28.1265 62.334064) (end 28.947186 63.15475) (width 0.2) (layer "B.Cu") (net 14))
 (segment (start 28.947186 63.15475) (end 31.115814 63.15475) (width 0.2) (layer "B.Cu") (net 14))
 (segment (start 28.1265 61.173436) (end 28.1265 62.334064) (width 0.2) (layer "B.Cu") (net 14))
 (segment (start 86.686691 40.948797) (end 83.90281 43.732678) (width 0.2) (layer "B.Cu") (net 13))
 (segment (start 89.513684 66.64475) (end 84.622684 61.75375) (width 0.2) (layer "B.Cu") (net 13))
 (segment (start 98.310691 40.342387) (end 98.310691 59.795375) (width 0.2) (layer "B.Cu") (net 13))
 (segment (start 79.8595 43.732678) (end 84.107381 39.484797) (width 0.2) (layer "B.Cu") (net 13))
 (segment (start 91.461316 66.64475) (end 89.513684 66.64475) (width 0.2) (layer "B.Cu") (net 13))
 (segment (start 84.107381 39.484797) (end 97.453101 39.484797) (width 0.2) (layer "B.Cu") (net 13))
 (segment (start 83.90281 43.732678) (end 79.8595 43.732678) (width 0.2) (layer "B.Cu") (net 13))
 (segment (start 98.310691 59.795375) (end 91.461316 66.64475) (width 0.2) (layer "B.Cu") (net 13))
 (segment (start 84.622684 61.75375) (end 67.31 61.75375) (width 0.2) (layer "B.Cu") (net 13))
 (segment (start 97.453101 39.484797) (end 98.310691 40.342387) (width 0.2) (layer "B.Cu") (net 13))
 (segment (start 97.909691 40.508487) (end 97.909691 56.312873) (width 0.2) (layer "B.Cu") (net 12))
 (segment (start 85.209691 39.885797) (end 97.287001 39.885797) (width 0.2) (layer "B.Cu") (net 12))
 (segment (start 84.146691 40.948797) (end 85.209691 39.885797) (width 0.2) (layer "B.Cu") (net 12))
 (segment (start 92.468814 61.75375) (end 86.6775 61.75375) (width 0.2) (layer "B.Cu") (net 12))
 (segment (start 97.909691 56.312873) (end 92.468814 61.75375) (width 0.2) (layer "B.Cu") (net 12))
 (segment (start 97.287001 39.885797) (end 97.909691 40.508487) (width 0.2) (layer "B.Cu") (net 12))
 (segment (start 49.86875 50.825) (end 38.91875 50.825) (width 0.2) (layer "F.Cu") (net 18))
 (segment (start 38.91875 50.825) (end 35.71875 47.625) (width 0.2) (layer "F.Cu") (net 18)))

